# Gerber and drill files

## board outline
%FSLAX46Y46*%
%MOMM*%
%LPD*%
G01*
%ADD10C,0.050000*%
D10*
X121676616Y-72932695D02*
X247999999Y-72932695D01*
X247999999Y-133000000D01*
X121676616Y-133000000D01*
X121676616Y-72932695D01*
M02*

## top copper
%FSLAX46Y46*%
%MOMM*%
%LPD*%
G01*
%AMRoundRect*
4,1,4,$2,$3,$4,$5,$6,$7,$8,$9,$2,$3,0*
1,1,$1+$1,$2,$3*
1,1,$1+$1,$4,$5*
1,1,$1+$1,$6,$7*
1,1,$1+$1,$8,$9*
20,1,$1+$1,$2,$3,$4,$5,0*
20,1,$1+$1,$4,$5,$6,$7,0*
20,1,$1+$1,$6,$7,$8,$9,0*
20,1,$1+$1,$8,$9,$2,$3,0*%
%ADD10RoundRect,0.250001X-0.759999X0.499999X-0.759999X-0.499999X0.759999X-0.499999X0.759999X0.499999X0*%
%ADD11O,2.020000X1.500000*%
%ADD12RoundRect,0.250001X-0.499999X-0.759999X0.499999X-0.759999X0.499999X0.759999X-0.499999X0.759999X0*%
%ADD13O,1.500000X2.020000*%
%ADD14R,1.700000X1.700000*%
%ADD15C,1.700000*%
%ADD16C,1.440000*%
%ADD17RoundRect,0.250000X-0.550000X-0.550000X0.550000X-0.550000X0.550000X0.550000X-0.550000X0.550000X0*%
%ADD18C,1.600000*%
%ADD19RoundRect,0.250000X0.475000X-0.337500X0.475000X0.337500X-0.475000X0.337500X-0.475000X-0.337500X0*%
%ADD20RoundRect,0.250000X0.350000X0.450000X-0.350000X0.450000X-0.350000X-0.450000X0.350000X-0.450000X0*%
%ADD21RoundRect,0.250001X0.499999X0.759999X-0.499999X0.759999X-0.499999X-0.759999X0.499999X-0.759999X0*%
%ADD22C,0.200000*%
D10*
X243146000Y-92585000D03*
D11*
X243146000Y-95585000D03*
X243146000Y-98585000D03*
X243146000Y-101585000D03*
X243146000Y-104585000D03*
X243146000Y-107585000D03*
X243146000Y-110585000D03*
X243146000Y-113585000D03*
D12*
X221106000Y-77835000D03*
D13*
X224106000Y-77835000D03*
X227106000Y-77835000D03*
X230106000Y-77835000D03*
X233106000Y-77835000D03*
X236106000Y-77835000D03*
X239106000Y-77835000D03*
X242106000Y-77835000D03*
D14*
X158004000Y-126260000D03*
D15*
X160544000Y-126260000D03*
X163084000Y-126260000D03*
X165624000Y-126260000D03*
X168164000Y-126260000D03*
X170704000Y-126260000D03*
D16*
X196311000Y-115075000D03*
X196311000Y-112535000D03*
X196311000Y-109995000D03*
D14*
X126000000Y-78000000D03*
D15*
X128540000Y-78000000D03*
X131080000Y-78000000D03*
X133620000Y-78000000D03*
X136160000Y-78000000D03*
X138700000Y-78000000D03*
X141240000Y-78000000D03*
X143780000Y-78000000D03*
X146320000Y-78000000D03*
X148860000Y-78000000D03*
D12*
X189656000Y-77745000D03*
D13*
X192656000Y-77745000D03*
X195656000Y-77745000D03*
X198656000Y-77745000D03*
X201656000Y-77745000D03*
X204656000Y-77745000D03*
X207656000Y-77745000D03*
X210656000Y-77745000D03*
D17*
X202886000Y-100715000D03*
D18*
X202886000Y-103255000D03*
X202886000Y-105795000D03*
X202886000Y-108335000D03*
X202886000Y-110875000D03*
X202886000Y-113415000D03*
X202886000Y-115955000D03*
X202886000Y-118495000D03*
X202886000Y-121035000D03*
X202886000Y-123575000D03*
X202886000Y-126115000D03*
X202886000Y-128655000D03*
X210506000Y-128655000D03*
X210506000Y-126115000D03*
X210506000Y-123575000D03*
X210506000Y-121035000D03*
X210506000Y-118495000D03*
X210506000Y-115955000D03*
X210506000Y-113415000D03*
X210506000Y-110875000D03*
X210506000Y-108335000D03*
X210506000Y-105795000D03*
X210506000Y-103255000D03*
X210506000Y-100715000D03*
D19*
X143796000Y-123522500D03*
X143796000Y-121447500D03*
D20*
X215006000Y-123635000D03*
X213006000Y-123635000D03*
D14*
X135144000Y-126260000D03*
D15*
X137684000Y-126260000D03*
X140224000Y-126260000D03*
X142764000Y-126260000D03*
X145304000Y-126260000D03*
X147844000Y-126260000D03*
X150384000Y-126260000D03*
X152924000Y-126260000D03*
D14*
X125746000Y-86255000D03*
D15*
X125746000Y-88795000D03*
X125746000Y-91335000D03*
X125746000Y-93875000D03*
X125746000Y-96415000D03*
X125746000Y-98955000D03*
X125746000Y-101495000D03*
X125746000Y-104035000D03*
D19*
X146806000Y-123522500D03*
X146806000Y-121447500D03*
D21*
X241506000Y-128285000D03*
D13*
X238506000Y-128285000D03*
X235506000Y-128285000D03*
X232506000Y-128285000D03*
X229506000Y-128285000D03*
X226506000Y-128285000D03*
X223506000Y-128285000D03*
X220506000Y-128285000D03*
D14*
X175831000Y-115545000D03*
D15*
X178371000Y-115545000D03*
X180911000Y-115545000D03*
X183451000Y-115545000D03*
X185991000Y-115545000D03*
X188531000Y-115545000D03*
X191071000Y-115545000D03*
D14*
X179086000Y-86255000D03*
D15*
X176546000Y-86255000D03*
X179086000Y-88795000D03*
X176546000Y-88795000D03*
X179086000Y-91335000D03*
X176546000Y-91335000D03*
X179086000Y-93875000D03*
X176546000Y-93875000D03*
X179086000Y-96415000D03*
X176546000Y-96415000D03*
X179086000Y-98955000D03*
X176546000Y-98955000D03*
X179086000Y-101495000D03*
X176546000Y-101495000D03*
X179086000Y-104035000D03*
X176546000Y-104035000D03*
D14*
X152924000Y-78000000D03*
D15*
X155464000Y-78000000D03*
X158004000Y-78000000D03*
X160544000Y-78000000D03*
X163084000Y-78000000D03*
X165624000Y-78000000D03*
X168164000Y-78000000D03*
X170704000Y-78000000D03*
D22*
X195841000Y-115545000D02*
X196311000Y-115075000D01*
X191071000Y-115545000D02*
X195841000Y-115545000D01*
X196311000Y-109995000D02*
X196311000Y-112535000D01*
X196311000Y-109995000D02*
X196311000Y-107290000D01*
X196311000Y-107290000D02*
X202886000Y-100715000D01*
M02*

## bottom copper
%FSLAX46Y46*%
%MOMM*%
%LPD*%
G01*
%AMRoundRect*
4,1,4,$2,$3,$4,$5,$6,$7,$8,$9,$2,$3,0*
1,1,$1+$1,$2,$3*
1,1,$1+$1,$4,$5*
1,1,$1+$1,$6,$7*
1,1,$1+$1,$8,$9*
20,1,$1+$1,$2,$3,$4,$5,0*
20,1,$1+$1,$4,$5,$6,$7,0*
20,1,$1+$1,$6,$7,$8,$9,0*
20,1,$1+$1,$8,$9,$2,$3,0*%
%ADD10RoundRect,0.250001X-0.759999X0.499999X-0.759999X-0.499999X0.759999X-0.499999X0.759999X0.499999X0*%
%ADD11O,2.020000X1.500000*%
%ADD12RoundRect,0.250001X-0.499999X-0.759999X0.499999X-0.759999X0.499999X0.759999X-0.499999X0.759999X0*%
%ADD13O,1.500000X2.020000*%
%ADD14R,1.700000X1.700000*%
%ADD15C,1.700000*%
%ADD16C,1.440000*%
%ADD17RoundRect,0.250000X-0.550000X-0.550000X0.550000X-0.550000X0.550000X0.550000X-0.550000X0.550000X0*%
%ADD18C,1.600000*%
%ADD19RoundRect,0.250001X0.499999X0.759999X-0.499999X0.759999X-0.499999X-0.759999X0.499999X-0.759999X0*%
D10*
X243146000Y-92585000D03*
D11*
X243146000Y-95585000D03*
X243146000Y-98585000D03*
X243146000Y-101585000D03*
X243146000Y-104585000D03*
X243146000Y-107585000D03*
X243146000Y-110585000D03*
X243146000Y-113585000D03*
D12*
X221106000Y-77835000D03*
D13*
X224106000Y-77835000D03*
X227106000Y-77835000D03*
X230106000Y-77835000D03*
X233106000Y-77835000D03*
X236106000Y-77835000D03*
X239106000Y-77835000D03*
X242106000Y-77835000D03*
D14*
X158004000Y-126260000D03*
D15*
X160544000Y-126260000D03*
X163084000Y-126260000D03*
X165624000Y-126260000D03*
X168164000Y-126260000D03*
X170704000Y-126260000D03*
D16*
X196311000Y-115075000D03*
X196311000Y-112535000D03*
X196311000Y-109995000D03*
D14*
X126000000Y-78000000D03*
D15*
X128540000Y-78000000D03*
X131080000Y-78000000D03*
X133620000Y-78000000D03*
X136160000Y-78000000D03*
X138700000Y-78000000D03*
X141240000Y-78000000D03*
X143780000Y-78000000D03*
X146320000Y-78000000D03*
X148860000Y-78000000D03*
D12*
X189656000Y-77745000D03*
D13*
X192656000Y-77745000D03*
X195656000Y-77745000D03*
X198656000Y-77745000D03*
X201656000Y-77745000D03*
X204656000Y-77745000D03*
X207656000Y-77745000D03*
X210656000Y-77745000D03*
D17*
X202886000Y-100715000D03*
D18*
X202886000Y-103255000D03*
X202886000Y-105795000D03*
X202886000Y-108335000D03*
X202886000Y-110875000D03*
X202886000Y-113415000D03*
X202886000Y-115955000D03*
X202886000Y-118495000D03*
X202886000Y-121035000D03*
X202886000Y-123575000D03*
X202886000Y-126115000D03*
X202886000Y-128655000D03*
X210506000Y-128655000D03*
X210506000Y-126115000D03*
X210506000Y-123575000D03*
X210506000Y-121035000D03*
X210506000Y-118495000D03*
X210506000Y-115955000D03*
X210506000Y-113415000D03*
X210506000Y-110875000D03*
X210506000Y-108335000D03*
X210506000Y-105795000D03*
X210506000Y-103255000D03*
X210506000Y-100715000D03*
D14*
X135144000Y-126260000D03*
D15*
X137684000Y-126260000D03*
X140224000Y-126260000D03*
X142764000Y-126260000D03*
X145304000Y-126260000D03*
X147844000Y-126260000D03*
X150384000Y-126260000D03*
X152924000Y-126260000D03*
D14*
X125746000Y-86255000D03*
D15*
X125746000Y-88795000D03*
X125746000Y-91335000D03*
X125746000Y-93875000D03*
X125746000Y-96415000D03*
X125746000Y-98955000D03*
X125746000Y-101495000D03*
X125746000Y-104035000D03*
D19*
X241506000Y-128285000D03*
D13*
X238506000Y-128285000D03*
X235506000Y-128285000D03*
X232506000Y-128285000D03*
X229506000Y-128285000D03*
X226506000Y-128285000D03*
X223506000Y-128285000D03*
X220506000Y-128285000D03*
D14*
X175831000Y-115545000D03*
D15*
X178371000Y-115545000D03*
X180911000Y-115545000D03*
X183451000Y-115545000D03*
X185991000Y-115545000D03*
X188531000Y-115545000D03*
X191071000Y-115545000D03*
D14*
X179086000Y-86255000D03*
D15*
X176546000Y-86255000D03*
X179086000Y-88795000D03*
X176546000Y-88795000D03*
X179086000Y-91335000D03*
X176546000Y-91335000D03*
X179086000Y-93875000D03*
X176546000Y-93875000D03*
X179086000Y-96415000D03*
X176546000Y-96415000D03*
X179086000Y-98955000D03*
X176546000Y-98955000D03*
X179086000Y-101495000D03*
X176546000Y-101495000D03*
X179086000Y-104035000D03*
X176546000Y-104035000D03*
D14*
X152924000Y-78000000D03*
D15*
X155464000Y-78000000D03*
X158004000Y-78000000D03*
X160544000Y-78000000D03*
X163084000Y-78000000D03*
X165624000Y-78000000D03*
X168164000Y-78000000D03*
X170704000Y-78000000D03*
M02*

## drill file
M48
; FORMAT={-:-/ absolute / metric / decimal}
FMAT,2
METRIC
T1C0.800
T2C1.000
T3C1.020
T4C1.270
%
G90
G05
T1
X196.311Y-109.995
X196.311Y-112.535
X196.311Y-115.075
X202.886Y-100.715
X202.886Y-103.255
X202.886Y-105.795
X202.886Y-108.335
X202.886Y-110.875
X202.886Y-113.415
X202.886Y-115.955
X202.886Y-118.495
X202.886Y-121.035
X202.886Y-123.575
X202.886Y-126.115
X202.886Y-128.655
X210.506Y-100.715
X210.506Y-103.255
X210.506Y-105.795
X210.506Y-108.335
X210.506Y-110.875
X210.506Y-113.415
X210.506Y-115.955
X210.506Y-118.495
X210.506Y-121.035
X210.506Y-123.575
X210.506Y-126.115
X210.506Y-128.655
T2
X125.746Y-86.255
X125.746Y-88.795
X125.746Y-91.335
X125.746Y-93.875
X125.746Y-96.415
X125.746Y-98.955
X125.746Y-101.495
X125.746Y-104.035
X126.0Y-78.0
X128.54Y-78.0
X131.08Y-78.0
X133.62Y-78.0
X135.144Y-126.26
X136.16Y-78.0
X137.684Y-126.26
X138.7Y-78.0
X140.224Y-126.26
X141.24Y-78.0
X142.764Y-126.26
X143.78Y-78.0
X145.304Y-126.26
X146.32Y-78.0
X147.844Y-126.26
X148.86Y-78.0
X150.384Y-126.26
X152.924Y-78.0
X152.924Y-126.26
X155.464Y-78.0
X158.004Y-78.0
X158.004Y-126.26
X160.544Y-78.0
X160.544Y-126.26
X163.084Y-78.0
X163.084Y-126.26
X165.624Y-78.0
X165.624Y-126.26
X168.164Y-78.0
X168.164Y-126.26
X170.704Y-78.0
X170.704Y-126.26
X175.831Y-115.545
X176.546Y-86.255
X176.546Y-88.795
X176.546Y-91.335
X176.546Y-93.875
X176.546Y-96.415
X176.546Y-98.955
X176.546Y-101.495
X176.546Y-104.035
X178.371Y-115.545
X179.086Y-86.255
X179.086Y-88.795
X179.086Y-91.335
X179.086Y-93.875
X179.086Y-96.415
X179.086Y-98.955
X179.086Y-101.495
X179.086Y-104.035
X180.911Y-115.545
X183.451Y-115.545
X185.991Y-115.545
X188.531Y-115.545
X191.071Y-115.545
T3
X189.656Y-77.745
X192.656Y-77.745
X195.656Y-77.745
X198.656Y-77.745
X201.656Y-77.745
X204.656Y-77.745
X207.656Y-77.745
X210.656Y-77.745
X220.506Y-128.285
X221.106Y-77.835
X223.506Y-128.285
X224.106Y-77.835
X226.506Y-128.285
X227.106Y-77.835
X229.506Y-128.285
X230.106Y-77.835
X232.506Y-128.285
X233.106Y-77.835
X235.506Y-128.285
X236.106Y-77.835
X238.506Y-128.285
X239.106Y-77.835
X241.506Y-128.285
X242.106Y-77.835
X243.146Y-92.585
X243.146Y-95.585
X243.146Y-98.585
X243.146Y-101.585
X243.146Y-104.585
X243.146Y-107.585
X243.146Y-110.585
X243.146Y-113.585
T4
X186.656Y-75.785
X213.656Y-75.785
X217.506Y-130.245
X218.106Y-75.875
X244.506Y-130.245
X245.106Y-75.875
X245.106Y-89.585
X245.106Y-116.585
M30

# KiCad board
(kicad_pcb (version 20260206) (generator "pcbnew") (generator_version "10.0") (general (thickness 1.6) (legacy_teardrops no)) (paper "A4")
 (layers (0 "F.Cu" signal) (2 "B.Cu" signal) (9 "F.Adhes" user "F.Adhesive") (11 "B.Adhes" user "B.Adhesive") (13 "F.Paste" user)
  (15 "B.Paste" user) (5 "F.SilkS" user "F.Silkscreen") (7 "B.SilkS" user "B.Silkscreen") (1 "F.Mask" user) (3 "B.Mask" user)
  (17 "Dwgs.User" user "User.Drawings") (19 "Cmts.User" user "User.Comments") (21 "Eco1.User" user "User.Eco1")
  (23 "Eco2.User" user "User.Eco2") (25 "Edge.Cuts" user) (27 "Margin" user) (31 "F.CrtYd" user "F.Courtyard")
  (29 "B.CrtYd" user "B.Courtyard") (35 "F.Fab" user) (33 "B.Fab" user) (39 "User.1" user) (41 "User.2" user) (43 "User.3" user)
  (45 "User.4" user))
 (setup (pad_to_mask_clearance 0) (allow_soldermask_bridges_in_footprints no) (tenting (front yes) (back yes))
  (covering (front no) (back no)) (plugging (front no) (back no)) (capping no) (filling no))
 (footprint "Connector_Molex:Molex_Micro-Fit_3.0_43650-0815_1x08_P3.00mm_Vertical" (layer "F.Cu") (at 243.146 92.585 -90)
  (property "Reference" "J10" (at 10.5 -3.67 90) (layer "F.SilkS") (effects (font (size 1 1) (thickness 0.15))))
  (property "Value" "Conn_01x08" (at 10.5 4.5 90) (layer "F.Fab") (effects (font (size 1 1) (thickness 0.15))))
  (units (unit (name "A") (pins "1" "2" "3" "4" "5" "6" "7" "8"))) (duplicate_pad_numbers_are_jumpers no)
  (pad "" np_thru_hole circle (at -3 -1.96 270) (size 1.27 1.27) (drill 1.27) (layers "*.Cu" "*.Mask"))
  (pad "" np_thru_hole circle (at 24 -1.96 270) (size 1.27 1.27) (drill 1.27) (layers "*.Cu" "*.Mask"))
  (pad "1" thru_hole roundrect (at 0 0 270) (size 1.5 2.02) (drill 1.02) (layers "*.Cu" "*.Mask") (remove_unused_layers no)
   (roundrect_rratio 0.166667) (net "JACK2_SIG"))
  (pad "2" thru_hole oval (at 3 0 270) (size 1.5 2.02) (drill 1.02) (layers "*.Cu" "*.Mask") (remove_unused_layers no) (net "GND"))
  (pad "3" thru_hole oval (at 6 0 270) (size 1.5 2.02) (drill 1.02) (layers "*.Cu" "*.Mask") (remove_unused_layers no) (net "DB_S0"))
  (pad "4" thru_hole oval (at 9 0 270) (size 1.5 2.02) (drill 1.02) (layers "*.Cu" "*.Mask") (remove_unused_layers no) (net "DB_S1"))
  (pad "5" thru_hole oval (at 12 0 270) (size 1.5 2.02) (drill 1.02) (layers "*.Cu" "*.Mask") (remove_unused_layers no) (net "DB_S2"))
  (pad "6" thru_hole oval (at 15 0 270) (size 1.5 2.02) (drill 1.02) (layers "*.Cu" "*.Mask") (remove_unused_layers no) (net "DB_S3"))
  (pad "7" thru_hole oval (at 18 0 270) (size 1.5 2.02) (drill 1.02) (layers "*.Cu" "*.Mask") (remove_unused_layers no) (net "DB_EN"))
  (pad "8" thru_hole oval (at 21 0 270) (size 1.5 2.02) (drill 1.02) (layers "*.Cu" "*.Mask") (remove_unused_layers no) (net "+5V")))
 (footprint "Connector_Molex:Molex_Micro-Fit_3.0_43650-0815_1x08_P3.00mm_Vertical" (layer "F.Cu") (at 221.106 77.835)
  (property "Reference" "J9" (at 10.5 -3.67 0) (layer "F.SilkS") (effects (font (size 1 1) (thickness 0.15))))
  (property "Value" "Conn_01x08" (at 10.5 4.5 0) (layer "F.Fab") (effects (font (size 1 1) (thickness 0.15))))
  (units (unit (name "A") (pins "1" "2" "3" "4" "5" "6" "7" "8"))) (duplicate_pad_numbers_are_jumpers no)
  (pad "" np_thru_hole circle (at -3 -1.96) (size 1.27 1.27) (drill 1.27) (layers "*.Cu" "*.Mask"))
  (pad "" np_thru_hole circle (at 24 -1.96) (size 1.27 1.27) (drill 1.27) (layers "*.Cu" "*.Mask"))
  (pad "1" thru_hole roundrect (at 0 0) (size 1.5 2.02) (drill 1.02) (layers "*.Cu" "*.Mask") (remove_unused_layers no)
   (roundrect_rratio 0.166667) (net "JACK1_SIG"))
  (pad "2" thru_hole oval (at 3 0) (size 1.5 2.02) (drill 1.02) (layers "*.Cu" "*.Mask") (remove_unused_layers no) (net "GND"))
  (pad "3" thru_hole oval (at 6 0) (size 1.5 2.02) (drill 1.02) (layers "*.Cu" "*.Mask") (remove_unused_layers no) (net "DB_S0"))
  (pad "4" thru_hole oval (at 9 0) (size 1.5 2.02) (drill 1.02) (layers "*.Cu" "*.Mask") (remove_unused_layers no) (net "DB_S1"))
  (pad "5" thru_hole oval (at 12 0) (size 1.5 2.02) (drill 1.02) (layers "*.Cu" "*.Mask") (remove_unused_layers no) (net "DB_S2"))
  (pad "6" thru_hole oval (at 15 0) (size 1.5 2.02) (drill 1.02) (layers "*.Cu" "*.Mask") (remove_unused_layers no) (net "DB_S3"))
  (pad "7" thru_hole oval (at 18 0) (size 1.5 2.02) (drill 1.02) (layers "*.Cu" "*.Mask") (remove_unused_layers no) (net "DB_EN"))
  (pad "8" thru_hole oval (at 21 0) (size 1.5 2.02) (drill 1.02) (layers "*.Cu" "*.Mask") (remove_unused_layers no) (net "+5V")))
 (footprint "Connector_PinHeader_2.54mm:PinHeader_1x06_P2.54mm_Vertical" (layer "F.Cu") (at 158.004 126.26 90)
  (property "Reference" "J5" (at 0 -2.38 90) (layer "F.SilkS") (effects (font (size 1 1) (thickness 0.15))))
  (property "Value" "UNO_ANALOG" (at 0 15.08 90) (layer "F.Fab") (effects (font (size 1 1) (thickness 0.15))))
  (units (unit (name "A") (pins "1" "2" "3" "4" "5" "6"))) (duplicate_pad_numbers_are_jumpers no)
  (pad "1" thru_hole rect (at 0 0 90) (size 1.7 1.7) (drill 1) (layers "*.Cu" "*.Mask") (remove_unused_layers no) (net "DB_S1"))
  (pad "2" thru_hole circle (at 0 2.54 90) (size 1.7 1.7) (drill 1) (layers "*.Cu" "*.Mask") (remove_unused_layers no) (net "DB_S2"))
  (pad "3" thru_hole circle (at 0 5.08 90) (size 1.7 1.7) (drill 1) (layers "*.Cu" "*.Mask") (remove_unused_layers no) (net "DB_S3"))
  (pad "4" thru_hole circle (at 0 7.62 90) (size 1.7 1.7) (drill 1) (layers "*.Cu" "*.Mask") (remove_unused_layers no) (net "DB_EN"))
  (pad "5" thru_hole circle (at 0 10.16 90) (size 1.7 1.7) (drill 1) (layers "*.Cu" "*.Mask") (remove_unused_layers no)
   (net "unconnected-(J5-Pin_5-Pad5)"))
  (pad "6" thru_hole circle (at 0 12.7 90) (size 1.7 1.7) (drill 1) (layers "*.Cu" "*.Mask") (remove_unused_layers no)
   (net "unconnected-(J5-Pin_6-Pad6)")))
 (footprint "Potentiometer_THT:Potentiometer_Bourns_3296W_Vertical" (layer "F.Cu") (at 196.311 115.075 -90)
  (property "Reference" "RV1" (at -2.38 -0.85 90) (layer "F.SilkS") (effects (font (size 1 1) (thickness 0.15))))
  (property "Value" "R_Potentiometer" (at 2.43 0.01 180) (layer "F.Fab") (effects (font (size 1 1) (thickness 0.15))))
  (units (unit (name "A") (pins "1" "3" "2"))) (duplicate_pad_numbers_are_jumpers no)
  (pad "1" thru_hole circle (at 0 0 270) (size 1.44 1.44) (drill 0.8) (layers "*.Cu" "*.Mask") (remove_unused_layers no) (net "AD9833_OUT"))
  (pad "2" thru_hole circle (at -2.54 0 270) (size 1.44 1.44) (drill 0.8) (layers "*.Cu" "*.Mask") (remove_unused_layers no)
   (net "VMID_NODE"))
  (pad "3" thru_hole circle (at -5.08 0 270) (size 1.44 1.44) (drill 0.8) (layers "*.Cu" "*.Mask") (remove_unused_layers no)
   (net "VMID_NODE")))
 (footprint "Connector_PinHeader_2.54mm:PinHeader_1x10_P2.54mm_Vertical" (layer "F.Cu") (at 126 78 90)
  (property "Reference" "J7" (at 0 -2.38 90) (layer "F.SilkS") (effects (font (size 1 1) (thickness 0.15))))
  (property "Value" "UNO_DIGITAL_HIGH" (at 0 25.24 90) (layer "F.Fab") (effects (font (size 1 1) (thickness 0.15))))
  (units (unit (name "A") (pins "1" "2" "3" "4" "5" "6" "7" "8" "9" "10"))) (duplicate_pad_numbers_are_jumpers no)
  (pad "1" thru_hole rect (at 0 0 90) (size 1.7 1.7) (drill 1) (layers "*.Cu" "*.Mask") (remove_unused_layers no) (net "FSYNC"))
  (pad "2" thru_hole circle (at 0 2.54 90) (size 1.7 1.7) (drill 1) (layers "*.Cu" "*.Mask") (remove_unused_layers no) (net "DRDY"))
  (pad "3" thru_hole circle (at 0 5.08 90) (size 1.7 1.7) (drill 1) (layers "*.Cu" "*.Mask") (remove_unused_layers no) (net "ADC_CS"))
  (pad "4" thru_hole circle (at 0 7.62 90) (size 1.7 1.7) (drill 1) (layers "*.Cu" "*.Mask") (remove_unused_layers no) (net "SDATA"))
  (pad "5" thru_hole circle (at 0 10.16 90) (size 1.7 1.7) (drill 1) (layers "*.Cu" "*.Mask") (remove_unused_layers no) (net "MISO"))
  (pad "6" thru_hole circle (at 0 12.7 90) (size 1.7 1.7) (drill 1) (layers "*.Cu" "*.Mask") (remove_unused_layers no) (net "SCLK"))
  (pad "7" thru_hole circle (at 0 15.24 90) (size 1.7 1.7) (drill 1) (layers "*.Cu" "*.Mask") (remove_unused_layers no) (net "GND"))
  (pad "8" thru_hole circle (at 0 17.78 90) (size 1.7 1.7) (drill 1) (layers "*.Cu" "*.Mask") (remove_unused_layers no)
   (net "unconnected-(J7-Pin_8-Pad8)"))
  (pad "9" thru_hole circle (at 0 20.32 90) (size 1.7 1.7) (drill 1) (layers "*.Cu" "*.Mask") (remove_unused_layers no)
   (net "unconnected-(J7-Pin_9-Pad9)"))
  (pad "10" thru_hole circle (at 0 22.86 90) (size 1.7 1.7) (drill 1) (layers "*.Cu" "*.Mask") (remove_unused_layers no)
   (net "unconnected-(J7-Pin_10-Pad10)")))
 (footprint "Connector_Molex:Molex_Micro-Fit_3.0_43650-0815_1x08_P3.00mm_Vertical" (layer "F.Cu") (at 189.656 77.745)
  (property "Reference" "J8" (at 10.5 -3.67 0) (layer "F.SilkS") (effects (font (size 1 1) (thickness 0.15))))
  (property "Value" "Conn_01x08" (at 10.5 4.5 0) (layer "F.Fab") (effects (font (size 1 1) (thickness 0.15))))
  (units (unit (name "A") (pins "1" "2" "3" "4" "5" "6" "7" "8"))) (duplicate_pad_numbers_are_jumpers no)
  (pad "" np_thru_hole circle (at -3 -1.96) (size 1.27 1.27) (drill 1.27) (layers "*.Cu" "*.Mask"))
  (pad "" np_thru_hole circle (at 24 -1.96) (size 1.27 1.27) (drill 1.27) (layers "*.Cu" "*.Mask"))
  (pad "1" thru_hole roundrect (at 0 0) (size 1.5 2.02) (drill 1.02) (layers "*.Cu" "*.Mask") (remove_unused_layers no)
   (roundrect_rratio 0.166667) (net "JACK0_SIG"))
  (pad "2" thru_hole oval (at 3 0) (size 1.5 2.02) (drill 1.02) (layers "*.Cu" "*.Mask") (remove_unused_layers no) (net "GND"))
  (pad "3" thru_hole oval (at 6 0) (size 1.5 2.02) (drill 1.02) (layers "*.Cu" "*.Mask") (remove_unused_layers no) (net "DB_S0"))
  (pad "4" thru_hole oval (at 9 0) (size 1.5 2.02) (drill 1.02) (layers "*.Cu" "*.Mask") (remove_unused_layers no) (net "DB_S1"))
  (pad "5" thru_hole oval (at 12 0) (size 1.5 2.02) (drill 1.02) (layers "*.Cu" "*.Mask") (remove_unused_layers no) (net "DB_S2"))
  (pad "6" thru_hole oval (at 15 0) (size 1.5 2.02) (drill 1.02) (layers "*.Cu" "*.Mask") (remove_unused_layers no) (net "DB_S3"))
  (pad "7" thru_hole oval (at 18 0) (size 1.5 2.02) (drill 1.02) (layers "*.Cu" "*.Mask") (remove_unused_layers no) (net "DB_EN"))
  (pad "8" thru_hole oval (at 21 0) (size 1.5 2.02) (drill 1.02) (layers "*.Cu" "*.Mask") (remove_unused_layers no) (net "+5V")))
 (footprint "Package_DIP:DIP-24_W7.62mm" (layer "F.Cu") (at 202.886 100.715)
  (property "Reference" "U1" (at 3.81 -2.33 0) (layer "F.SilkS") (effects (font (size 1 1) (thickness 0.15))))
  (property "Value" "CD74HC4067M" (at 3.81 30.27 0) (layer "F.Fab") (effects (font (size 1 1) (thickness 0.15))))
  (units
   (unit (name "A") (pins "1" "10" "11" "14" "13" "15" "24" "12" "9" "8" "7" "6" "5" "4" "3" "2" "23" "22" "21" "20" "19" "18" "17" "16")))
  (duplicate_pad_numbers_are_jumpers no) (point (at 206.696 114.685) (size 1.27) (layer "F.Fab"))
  (pad "1" thru_hole roundrect (at 0 0) (size 1.6 1.6) (drill 0.8) (layers "*.Cu" "*.Mask") (remove_unused_layers no)
   (roundrect_rratio 0.15625) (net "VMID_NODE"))
  (pad "2" thru_hole circle (at 0 2.54) (size 1.6 1.6) (drill 0.8) (layers "*.Cu" "*.Mask") (remove_unused_layers no)
   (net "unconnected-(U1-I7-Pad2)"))
  (pad "3" thru_hole circle (at 0 5.08) (size 1.6 1.6) (drill 0.8) (layers "*.Cu" "*.Mask") (remove_unused_layers no)
   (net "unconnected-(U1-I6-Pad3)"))
  (pad "4" thru_hole circle (at 0 7.62) (size 1.6 1.6) (drill 0.8) (layers "*.Cu" "*.Mask") (remove_unused_layers no)
   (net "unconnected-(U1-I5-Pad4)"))
  (pad "5" thru_hole circle (at 0 10.16) (size 1.6 1.6) (drill 0.8) (layers "*.Cu" "*.Mask") (remove_unused_layers no)
   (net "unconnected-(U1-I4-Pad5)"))
  (pad "6" thru_hole circle (at 0 12.7) (size 1.6 1.6) (drill 0.8) (layers "*.Cu" "*.Mask") (remove_unused_layers no)
   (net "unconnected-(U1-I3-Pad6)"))
  (pad "7" thru_hole circle (at 0 15.24) (size 1.6 1.6) (drill 0.8) (layers "*.Cu" "*.Mask") (remove_unused_layers no)
   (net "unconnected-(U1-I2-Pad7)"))
  (pad "8" thru_hole circle (at 0 17.78) (size 1.6 1.6) (drill 0.8) (layers "*.Cu" "*.Mask") (remove_unused_layers no)
   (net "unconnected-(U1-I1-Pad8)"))
  (pad "9" thru_hole circle (at 0 20.32) (size 1.6 1.6) (drill 0.8) (layers "*.Cu" "*.Mask") (remove_unused_layers no)
   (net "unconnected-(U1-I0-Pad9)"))
  (pad "10" thru_hole circle (at 0 22.86) (size 1.6 1.6) (drill 0.8) (layers "*.Cu" "*.Mask") (remove_unused_layers no) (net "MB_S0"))
  (pad "11" thru_hole circle (at 0 25.4) (size 1.6 1.6) (drill 0.8) (layers "*.Cu" "*.Mask") (remove_unused_layers no) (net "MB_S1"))
  (pad "12" thru_hole circle (at 0 27.94) (size 1.6 1.6) (drill 0.8) (layers "*.Cu" "*.Mask") (remove_unused_layers no) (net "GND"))
  (pad "13" thru_hole circle (at 7.62 27.94) (size 1.6 1.6) (drill 0.8) (layers "*.Cu" "*.Mask") (remove_unused_layers no) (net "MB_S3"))
  (pad "14" thru_hole circle (at 7.62 25.4) (size 1.6 1.6) (drill 0.8) (layers "*.Cu" "*.Mask") (remove_unused_layers no) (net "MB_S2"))
  (pad "15" thru_hole circle (at 7.62 22.86) (size 1.6 1.6) (drill 0.8) (layers "*.Cu" "*.Mask") (remove_unused_layers no) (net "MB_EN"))
  (pad "16" thru_hole circle (at 7.62 20.32) (size 1.6 1.6) (drill 0.8) (layers "*.Cu" "*.Mask") (remove_unused_layers no)
   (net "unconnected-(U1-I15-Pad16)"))
  (pad "17" thru_hole circle (at 7.62 17.78) (size 1.6 1.6) (drill 0.8) (layers "*.Cu" "*.Mask") (remove_unused_layers no)
   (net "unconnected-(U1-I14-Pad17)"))
  (pad "18" thru_hole circle (at 7.62 15.24) (size 1.6 1.6) (drill 0.8) (layers "*.Cu" "*.Mask") (remove_unused_layers no)
   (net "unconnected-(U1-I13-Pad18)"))
  (pad "19" thru_hole circle (at 7.62 12.7) (size 1.6 1.6) (drill 0.8) (layers "*.Cu" "*.Mask") (remove_unused_layers no)
   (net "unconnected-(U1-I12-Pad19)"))
  (pad "20" thru_hole circle (at 7.62 10.16) (size 1.6 1.6) (drill 0.8) (layers "*.Cu" "*.Mask") (remove_unused_layers no) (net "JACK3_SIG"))
  (pad "21" thru_hole circle (at 7.62 7.62) (size 1.6 1.6) (drill 0.8) (layers "*.Cu" "*.Mask") (remove_unused_layers no) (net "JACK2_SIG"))
  (pad "22" thru_hole circle (at 7.62 5.08) (size 1.6 1.6) (drill 0.8) (layers "*.Cu" "*.Mask") (remove_unused_layers no) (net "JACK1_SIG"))
  (pad "23" thru_hole circle (at 7.62 2.54) (size 1.6 1.6) (drill 0.8) (layers "*.Cu" "*.Mask") (remove_unused_layers no) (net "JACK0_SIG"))
  (pad "24" thru_hole circle (at 7.62 0) (size 1.6 1.6) (drill 0.8) (layers "*.Cu" "*.Mask") (remove_unused_layers no) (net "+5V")))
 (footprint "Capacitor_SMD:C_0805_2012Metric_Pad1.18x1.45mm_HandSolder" (layer "F.Cu") (at 143.796 122.485 90)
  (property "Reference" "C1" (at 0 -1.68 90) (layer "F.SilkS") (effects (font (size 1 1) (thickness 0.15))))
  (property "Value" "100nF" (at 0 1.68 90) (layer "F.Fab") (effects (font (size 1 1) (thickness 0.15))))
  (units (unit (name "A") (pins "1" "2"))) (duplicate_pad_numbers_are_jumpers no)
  (pad "1" smd roundrect (at -1.0375 0 90) (size 1.175 1.45) (layers "F.Cu" "F.Mask" "F.Paste") (roundrect_rratio 0.212766) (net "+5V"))
  (pad "2" smd roundrect (at 1.0375 0 90) (size 1.175 1.45) (layers "F.Cu" "F.Mask" "F.Paste") (roundrect_rratio 0.212766) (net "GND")))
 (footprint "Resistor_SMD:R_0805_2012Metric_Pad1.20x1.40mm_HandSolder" (layer "F.Cu") (at 214.006 123.635 180)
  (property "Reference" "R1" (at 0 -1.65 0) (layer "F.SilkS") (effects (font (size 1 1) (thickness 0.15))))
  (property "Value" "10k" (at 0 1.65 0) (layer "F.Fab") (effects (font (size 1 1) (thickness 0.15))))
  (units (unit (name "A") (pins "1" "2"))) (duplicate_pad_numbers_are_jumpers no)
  (pad "1" smd roundrect (at -1 0 180) (size 1.2 1.4) (layers "F.Cu" "F.Mask" "F.Paste") (roundrect_rratio 0.208333) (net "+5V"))
  (pad "2" smd roundrect (at 1 0 180) (size 1.2 1.4) (layers "F.Cu" "F.Mask" "F.Paste") (roundrect_rratio 0.208333) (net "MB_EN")))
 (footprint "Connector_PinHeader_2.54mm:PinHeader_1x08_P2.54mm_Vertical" (layer "F.Cu") (at 135.144 126.26 90)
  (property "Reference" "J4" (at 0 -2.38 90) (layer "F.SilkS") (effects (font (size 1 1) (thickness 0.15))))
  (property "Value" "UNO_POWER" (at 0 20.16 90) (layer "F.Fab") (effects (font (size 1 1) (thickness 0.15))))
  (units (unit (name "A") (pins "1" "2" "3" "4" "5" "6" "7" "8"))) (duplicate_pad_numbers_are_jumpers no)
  (pad "1" thru_hole rect (at 0 0 90) (size 1.7 1.7) (drill 1) (layers "*.Cu" "*.Mask") (remove_unused_layers no)
   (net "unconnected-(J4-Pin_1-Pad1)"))
  (pad "2" thru_hole circle (at 0 2.54 90) (size 1.7 1.7) (drill 1) (layers "*.Cu" "*.Mask") (remove_unused_layers no)
   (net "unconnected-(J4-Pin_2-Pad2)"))
  (pad "3" thru_hole circle (at 0 5.08 90) (size 1.7 1.7) (drill 1) (layers "*.Cu" "*.Mask") (remove_unused_layers no)
   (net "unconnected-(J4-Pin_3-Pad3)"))
  (pad "4" thru_hole circle (at 0 7.62 90) (size 1.7 1.7) (drill 1) (layers "*.Cu" "*.Mask") (remove_unused_layers no)
   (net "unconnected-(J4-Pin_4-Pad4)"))
  (pad "5" thru_hole circle (at 0 10.16 90) (size 1.7 1.7) (drill 1) (layers "*.Cu" "*.Mask") (remove_unused_layers no) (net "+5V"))
  (pad "6" thru_hole circle (at 0 12.7 90) (size 1.7 1.7) (drill 1) (layers "*.Cu" "*.Mask") (remove_unused_layers no) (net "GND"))
  (pad "7" thru_hole circle (at 0 15.24 90) (size 1.7 1.7) (drill 1) (layers "*.Cu" "*.Mask") (remove_unused_layers no) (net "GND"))
  (pad "8" thru_hole circle (at 0 17.78 90) (size 1.7 1.7) (drill 1) (layers "*.Cu" "*.Mask") (remove_unused_layers no)
   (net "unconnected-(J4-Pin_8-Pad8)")))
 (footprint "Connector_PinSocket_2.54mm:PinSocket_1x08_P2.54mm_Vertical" (layer "F.Cu") (at 125.746 86.255)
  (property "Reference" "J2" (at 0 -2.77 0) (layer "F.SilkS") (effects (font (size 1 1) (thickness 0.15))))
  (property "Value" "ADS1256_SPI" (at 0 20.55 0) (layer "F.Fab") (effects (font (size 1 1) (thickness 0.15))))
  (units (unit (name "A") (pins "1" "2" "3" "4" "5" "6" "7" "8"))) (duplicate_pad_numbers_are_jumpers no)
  (pad "1" thru_hole rect (at 0 0) (size 1.7 1.7) (drill 1) (layers "*.Cu" "*.Mask") (remove_unused_layers no) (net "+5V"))
  (pad "2" thru_hole circle (at 0 2.54) (size 1.7 1.7) (drill 1) (layers "*.Cu" "*.Mask") (remove_unused_layers no) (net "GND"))
  (pad "3" thru_hole circle (at 0 5.08) (size 1.7 1.7) (drill 1) (layers "*.Cu" "*.Mask") (remove_unused_layers no) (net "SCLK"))
  (pad "4" thru_hole circle (at 0 7.62) (size 1.7 1.7) (drill 1) (layers "*.Cu" "*.Mask") (remove_unused_layers no) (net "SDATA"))
  (pad "5" thru_hole circle (at 0 10.16) (size 1.7 1.7) (drill 1) (layers "*.Cu" "*.Mask") (remove_unused_layers no) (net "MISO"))
  (pad "6" thru_hole circle (at 0 12.7) (size 1.7 1.7) (drill 1) (layers "*.Cu" "*.Mask") (remove_unused_layers no) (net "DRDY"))
  (pad "7" thru_hole circle (at 0 15.24) (size 1.7 1.7) (drill 1) (layers "*.Cu" "*.Mask") (remove_unused_layers no) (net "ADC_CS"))
  (pad "8" thru_hole circle (at 0 17.78) (size 1.7 1.7) (drill 1) (layers "*.Cu" "*.Mask") (remove_unused_layers no) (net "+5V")))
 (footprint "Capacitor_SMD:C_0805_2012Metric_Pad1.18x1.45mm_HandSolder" (layer "F.Cu") (at 146.806 122.485 90)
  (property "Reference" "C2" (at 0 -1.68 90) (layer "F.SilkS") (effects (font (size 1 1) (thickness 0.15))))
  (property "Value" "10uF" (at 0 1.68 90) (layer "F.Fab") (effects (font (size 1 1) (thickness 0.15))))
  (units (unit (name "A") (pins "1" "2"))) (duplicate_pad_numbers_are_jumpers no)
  (pad "1" smd roundrect (at -1.0375 0 90) (size 1.175 1.45) (layers "F.Cu" "F.Mask" "F.Paste") (roundrect_rratio 0.212766) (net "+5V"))
  (pad "2" smd roundrect (at 1.0375 0 90) (size 1.175 1.45) (layers "F.Cu" "F.Mask" "F.Paste") (roundrect_rratio 0.212766) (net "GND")))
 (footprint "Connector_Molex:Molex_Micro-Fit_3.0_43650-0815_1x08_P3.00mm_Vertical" (layer "F.Cu") (at 241.506 128.285 180)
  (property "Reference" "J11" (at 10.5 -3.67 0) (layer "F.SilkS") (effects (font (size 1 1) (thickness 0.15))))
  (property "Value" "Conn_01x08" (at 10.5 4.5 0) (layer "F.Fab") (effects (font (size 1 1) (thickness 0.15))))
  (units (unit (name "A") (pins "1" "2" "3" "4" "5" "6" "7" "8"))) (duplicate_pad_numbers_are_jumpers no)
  (pad "" np_thru_hole circle (at -3 -1.96 180) (size 1.27 1.27) (drill 1.27) (layers "*.Cu" "*.Mask"))
  (pad "" np_thru_hole circle (at 24 -1.96 180) (size 1.27 1.27) (drill 1.27) (layers "*.Cu" "*.Mask"))
  (pad "1" thru_hole roundrect (at 0 0 180) (size 1.5 2.02) (drill 1.02) (layers "*.Cu" "*.Mask") (remove_unused_layers no)
   (roundrect_rratio 0.166667) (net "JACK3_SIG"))
  (pad "2" thru_hole oval (at 3 0 180) (size 1.5 2.02) (drill 1.02) (layers "*.Cu" "*.Mask") (remove_unused_layers no) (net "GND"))
  (pad "3" thru_hole oval (at 6 0 180) (size 1.5 2.02) (drill 1.02) (layers "*.Cu" "*.Mask") (remove_unused_layers no) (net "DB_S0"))
  (pad "4" thru_hole oval (at 9 0 180) (size 1.5 2.02) (drill 1.02) (layers "*.Cu" "*.Mask") (remove_unused_layers no) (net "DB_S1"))
  (pad "5" thru_hole oval (at 12 0 180) (size 1.5 2.02) (drill 1.02) (layers "*.Cu" "*.Mask") (remove_unused_layers no) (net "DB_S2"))
  (pad "6" thru_hole oval (at 15 0 180) (size 1.5 2.02) (drill 1.02) (layers "*.Cu" "*.Mask") (remove_unused_layers no) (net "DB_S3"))
  (pad "7" thru_hole oval (at 18 0 180) (size 1.5 2.02) (drill 1.02) (layers "*.Cu" "*.Mask") (remove_unused_layers no) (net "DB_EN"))
  (pad "8" thru_hole oval (at 21 0 180) (size 1.5 2.02) (drill 1.02) (layers "*.Cu" "*.Mask") (remove_unused_layers no) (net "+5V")))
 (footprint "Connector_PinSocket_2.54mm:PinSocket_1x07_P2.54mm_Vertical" (layer "F.Cu") (at 175.831 115.545 90)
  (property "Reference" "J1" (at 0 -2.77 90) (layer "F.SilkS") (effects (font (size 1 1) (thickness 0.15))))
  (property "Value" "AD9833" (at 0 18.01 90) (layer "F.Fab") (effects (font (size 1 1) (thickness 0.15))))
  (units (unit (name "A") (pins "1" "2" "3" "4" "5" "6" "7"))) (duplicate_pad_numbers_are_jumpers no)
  (pad "1" thru_hole rect (at 0 0 90) (size 1.7 1.7) (drill 1) (layers "*.Cu" "*.Mask") (remove_unused_layers no) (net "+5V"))
  (pad "2" thru_hole circle (at 0 2.54 90) (size 1.7 1.7) (drill 1) (layers "*.Cu" "*.Mask") (remove_unused_layers no) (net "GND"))
  (pad "3" thru_hole circle (at 0 5.08 90) (size 1.7 1.7) (drill 1) (layers "*.Cu" "*.Mask") (remove_unused_layers no) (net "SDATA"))
  (pad "4" thru_hole circle (at 0 7.62 90) (size 1.7 1.7) (drill 1) (layers "*.Cu" "*.Mask") (remove_unused_layers no) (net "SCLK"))
  (pad "5" thru_hole circle (at 0 10.16 90) (size 1.7 1.7) (drill 1) (layers "*.Cu" "*.Mask") (remove_unused_layers no) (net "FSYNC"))
  (pad "6" thru_hole circle (at 0 12.7 90) (size 1.7 1.7) (drill 1) (layers "*.Cu" "*.Mask") (remove_unused_layers no) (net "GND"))
  (pad "7" thru_hole circle (at 0 15.24 90) (size 1.7 1.7) (drill 1) (layers "*.Cu" "*.Mask") (remove_unused_layers no) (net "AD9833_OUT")))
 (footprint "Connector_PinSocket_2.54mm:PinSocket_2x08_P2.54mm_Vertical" (layer "F.Cu") (at 179.086 86.255)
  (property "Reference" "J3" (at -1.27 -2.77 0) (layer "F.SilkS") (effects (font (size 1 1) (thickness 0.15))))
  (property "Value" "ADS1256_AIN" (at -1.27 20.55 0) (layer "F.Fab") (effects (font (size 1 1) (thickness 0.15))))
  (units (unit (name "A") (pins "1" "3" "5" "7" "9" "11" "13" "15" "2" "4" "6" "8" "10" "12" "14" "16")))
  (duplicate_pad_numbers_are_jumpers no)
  (pad "1" thru_hole rect (at 0 0) (size 1.7 1.7) (drill 1) (layers "*.Cu" "*.Mask") (remove_unused_layers no) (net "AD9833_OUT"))
  (pad "2" thru_hole circle (at -2.54 0) (size 1.7 1.7) (drill 1) (layers "*.Cu" "*.Mask") (remove_unused_layers no) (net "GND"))
  (pad "3" thru_hole circle (at 0 2.54) (size 1.7 1.7) (drill 1) (layers "*.Cu" "*.Mask") (remove_unused_layers no) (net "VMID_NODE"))
  (pad "4" thru_hole circle (at -2.54 2.54) (size 1.7 1.7) (drill 1) (layers "*.Cu" "*.Mask") (remove_unused_layers no) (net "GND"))
  (pad "5" thru_hole circle (at 0 5.08) (size 1.7 1.7) (drill 1) (layers "*.Cu" "*.Mask") (remove_unused_layers no) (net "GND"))
  (pad "6" thru_hole circle (at -2.54 5.08) (size 1.7 1.7) (drill 1) (layers "*.Cu" "*.Mask") (remove_unused_layers no) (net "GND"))
  (pad "7" thru_hole circle (at 0 7.62) (size 1.7 1.7) (drill 1) (layers "*.Cu" "*.Mask") (remove_unused_layers no) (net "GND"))
  (pad "8" thru_hole circle (at -2.54 7.62) (size 1.7 1.7) (drill 1) (layers "*.Cu" "*.Mask") (remove_unused_layers no) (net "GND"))
  (pad "9" thru_hole circle (at 0 10.16) (size 1.7 1.7) (drill 1) (layers "*.Cu" "*.Mask") (remove_unused_layers no) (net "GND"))
  (pad "10" thru_hole circle (at -2.54 10.16) (size 1.7 1.7) (drill 1) (layers "*.Cu" "*.Mask") (remove_unused_layers no) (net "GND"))
  (pad "11" thru_hole circle (at 0 12.7) (size 1.7 1.7) (drill 1) (layers "*.Cu" "*.Mask") (remove_unused_layers no) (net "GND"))
  (pad "12" thru_hole circle (at -2.54 12.7) (size 1.7 1.7) (drill 1) (layers "*.Cu" "*.Mask") (remove_unused_layers no) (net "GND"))
  (pad "13" thru_hole circle (at 0 15.24) (size 1.7 1.7) (drill 1) (layers "*.Cu" "*.Mask") (remove_unused_layers no) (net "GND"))
  (pad "14" thru_hole circle (at -2.54 15.24) (size 1.7 1.7) (drill 1) (layers "*.Cu" "*.Mask") (remove_unused_layers no) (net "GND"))
  (pad "15" thru_hole circle (at 0 17.78) (size 1.7 1.7) (drill 1) (layers "*.Cu" "*.Mask") (remove_unused_layers no) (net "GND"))
  (pad "16" thru_hole circle (at -2.54 17.78) (size 1.7 1.7) (drill 1) (layers "*.Cu" "*.Mask") (remove_unused_layers no) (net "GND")))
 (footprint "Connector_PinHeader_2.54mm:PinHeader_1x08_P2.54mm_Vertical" (layer "F.Cu") (at 152.924 78 90)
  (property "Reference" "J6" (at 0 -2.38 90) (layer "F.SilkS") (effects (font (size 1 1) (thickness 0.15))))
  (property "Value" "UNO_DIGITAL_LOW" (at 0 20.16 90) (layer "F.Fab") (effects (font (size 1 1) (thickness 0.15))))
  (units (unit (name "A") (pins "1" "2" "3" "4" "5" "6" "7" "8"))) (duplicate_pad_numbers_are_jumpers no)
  (pad "1" thru_hole rect (at 0 0 90) (size 1.7 1.7) (drill 1) (layers "*.Cu" "*.Mask") (remove_unused_layers no)
   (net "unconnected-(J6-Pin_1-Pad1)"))
  (pad "2" thru_hole circle (at 0 2.54 90) (size 1.7 1.7) (drill 1) (layers "*.Cu" "*.Mask") (remove_unused_layers no)
   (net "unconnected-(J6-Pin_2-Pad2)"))
  (pad "3" thru_hole circle (at 0 5.08 90) (size 1.7 1.7) (drill 1) (layers "*.Cu" "*.Mask") (remove_unused_layers no) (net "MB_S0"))
  (pad "4" thru_hole circle (at 0 7.62 90) (size 1.7 1.7) (drill 1) (layers "*.Cu" "*.Mask") (remove_unused_layers no) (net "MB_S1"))
  (pad "5" thru_hole circle (at 0 10.16 90) (size 1.7 1.7) (drill 1) (layers "*.Cu" "*.Mask") (remove_unused_layers no) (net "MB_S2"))
  (pad "6" thru_hole circle (at 0 12.7 90) (size 1.7 1.7) (drill 1) (layers "*.Cu" "*.Mask") (remove_unused_layers no) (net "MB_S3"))
  (pad "7" thru_hole circle (at 0 15.24 90) (size 1.7 1.7) (drill 1) (layers "*.Cu" "*.Mask") (remove_unused_layers no) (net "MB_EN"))
  (pad "8" thru_hole circle (at 0 17.78 90) (size 1.7 1.7) (drill 1) (layers "*.Cu" "*.Mask") (remove_unused_layers no) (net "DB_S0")))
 (gr_rect (start 121.676616 72.932695) (end 247.999999 133) (stroke (width 0.05) (type default)) (fill no) (layer "Edge.Cuts"))
 (segment (start 195.841 115.545) (end 196.311 115.075) (width 0.2) (layer "F.Cu") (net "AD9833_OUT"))
 (segment (start 191.071 115.545) (end 195.841 115.545) (width 0.2) (layer "F.Cu") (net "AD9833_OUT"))
 (segment (start 196.311 109.995) (end 196.311 112.535) (width 0.2) (layer "F.Cu") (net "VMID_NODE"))
 (segment (start 196.311 109.995) (end 196.311 107.29) (width 0.2) (layer "F.Cu") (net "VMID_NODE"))
 (segment (start 196.311 107.29) (end 202.886 100.715) (width 0.2) (layer "F.Cu") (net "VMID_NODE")))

